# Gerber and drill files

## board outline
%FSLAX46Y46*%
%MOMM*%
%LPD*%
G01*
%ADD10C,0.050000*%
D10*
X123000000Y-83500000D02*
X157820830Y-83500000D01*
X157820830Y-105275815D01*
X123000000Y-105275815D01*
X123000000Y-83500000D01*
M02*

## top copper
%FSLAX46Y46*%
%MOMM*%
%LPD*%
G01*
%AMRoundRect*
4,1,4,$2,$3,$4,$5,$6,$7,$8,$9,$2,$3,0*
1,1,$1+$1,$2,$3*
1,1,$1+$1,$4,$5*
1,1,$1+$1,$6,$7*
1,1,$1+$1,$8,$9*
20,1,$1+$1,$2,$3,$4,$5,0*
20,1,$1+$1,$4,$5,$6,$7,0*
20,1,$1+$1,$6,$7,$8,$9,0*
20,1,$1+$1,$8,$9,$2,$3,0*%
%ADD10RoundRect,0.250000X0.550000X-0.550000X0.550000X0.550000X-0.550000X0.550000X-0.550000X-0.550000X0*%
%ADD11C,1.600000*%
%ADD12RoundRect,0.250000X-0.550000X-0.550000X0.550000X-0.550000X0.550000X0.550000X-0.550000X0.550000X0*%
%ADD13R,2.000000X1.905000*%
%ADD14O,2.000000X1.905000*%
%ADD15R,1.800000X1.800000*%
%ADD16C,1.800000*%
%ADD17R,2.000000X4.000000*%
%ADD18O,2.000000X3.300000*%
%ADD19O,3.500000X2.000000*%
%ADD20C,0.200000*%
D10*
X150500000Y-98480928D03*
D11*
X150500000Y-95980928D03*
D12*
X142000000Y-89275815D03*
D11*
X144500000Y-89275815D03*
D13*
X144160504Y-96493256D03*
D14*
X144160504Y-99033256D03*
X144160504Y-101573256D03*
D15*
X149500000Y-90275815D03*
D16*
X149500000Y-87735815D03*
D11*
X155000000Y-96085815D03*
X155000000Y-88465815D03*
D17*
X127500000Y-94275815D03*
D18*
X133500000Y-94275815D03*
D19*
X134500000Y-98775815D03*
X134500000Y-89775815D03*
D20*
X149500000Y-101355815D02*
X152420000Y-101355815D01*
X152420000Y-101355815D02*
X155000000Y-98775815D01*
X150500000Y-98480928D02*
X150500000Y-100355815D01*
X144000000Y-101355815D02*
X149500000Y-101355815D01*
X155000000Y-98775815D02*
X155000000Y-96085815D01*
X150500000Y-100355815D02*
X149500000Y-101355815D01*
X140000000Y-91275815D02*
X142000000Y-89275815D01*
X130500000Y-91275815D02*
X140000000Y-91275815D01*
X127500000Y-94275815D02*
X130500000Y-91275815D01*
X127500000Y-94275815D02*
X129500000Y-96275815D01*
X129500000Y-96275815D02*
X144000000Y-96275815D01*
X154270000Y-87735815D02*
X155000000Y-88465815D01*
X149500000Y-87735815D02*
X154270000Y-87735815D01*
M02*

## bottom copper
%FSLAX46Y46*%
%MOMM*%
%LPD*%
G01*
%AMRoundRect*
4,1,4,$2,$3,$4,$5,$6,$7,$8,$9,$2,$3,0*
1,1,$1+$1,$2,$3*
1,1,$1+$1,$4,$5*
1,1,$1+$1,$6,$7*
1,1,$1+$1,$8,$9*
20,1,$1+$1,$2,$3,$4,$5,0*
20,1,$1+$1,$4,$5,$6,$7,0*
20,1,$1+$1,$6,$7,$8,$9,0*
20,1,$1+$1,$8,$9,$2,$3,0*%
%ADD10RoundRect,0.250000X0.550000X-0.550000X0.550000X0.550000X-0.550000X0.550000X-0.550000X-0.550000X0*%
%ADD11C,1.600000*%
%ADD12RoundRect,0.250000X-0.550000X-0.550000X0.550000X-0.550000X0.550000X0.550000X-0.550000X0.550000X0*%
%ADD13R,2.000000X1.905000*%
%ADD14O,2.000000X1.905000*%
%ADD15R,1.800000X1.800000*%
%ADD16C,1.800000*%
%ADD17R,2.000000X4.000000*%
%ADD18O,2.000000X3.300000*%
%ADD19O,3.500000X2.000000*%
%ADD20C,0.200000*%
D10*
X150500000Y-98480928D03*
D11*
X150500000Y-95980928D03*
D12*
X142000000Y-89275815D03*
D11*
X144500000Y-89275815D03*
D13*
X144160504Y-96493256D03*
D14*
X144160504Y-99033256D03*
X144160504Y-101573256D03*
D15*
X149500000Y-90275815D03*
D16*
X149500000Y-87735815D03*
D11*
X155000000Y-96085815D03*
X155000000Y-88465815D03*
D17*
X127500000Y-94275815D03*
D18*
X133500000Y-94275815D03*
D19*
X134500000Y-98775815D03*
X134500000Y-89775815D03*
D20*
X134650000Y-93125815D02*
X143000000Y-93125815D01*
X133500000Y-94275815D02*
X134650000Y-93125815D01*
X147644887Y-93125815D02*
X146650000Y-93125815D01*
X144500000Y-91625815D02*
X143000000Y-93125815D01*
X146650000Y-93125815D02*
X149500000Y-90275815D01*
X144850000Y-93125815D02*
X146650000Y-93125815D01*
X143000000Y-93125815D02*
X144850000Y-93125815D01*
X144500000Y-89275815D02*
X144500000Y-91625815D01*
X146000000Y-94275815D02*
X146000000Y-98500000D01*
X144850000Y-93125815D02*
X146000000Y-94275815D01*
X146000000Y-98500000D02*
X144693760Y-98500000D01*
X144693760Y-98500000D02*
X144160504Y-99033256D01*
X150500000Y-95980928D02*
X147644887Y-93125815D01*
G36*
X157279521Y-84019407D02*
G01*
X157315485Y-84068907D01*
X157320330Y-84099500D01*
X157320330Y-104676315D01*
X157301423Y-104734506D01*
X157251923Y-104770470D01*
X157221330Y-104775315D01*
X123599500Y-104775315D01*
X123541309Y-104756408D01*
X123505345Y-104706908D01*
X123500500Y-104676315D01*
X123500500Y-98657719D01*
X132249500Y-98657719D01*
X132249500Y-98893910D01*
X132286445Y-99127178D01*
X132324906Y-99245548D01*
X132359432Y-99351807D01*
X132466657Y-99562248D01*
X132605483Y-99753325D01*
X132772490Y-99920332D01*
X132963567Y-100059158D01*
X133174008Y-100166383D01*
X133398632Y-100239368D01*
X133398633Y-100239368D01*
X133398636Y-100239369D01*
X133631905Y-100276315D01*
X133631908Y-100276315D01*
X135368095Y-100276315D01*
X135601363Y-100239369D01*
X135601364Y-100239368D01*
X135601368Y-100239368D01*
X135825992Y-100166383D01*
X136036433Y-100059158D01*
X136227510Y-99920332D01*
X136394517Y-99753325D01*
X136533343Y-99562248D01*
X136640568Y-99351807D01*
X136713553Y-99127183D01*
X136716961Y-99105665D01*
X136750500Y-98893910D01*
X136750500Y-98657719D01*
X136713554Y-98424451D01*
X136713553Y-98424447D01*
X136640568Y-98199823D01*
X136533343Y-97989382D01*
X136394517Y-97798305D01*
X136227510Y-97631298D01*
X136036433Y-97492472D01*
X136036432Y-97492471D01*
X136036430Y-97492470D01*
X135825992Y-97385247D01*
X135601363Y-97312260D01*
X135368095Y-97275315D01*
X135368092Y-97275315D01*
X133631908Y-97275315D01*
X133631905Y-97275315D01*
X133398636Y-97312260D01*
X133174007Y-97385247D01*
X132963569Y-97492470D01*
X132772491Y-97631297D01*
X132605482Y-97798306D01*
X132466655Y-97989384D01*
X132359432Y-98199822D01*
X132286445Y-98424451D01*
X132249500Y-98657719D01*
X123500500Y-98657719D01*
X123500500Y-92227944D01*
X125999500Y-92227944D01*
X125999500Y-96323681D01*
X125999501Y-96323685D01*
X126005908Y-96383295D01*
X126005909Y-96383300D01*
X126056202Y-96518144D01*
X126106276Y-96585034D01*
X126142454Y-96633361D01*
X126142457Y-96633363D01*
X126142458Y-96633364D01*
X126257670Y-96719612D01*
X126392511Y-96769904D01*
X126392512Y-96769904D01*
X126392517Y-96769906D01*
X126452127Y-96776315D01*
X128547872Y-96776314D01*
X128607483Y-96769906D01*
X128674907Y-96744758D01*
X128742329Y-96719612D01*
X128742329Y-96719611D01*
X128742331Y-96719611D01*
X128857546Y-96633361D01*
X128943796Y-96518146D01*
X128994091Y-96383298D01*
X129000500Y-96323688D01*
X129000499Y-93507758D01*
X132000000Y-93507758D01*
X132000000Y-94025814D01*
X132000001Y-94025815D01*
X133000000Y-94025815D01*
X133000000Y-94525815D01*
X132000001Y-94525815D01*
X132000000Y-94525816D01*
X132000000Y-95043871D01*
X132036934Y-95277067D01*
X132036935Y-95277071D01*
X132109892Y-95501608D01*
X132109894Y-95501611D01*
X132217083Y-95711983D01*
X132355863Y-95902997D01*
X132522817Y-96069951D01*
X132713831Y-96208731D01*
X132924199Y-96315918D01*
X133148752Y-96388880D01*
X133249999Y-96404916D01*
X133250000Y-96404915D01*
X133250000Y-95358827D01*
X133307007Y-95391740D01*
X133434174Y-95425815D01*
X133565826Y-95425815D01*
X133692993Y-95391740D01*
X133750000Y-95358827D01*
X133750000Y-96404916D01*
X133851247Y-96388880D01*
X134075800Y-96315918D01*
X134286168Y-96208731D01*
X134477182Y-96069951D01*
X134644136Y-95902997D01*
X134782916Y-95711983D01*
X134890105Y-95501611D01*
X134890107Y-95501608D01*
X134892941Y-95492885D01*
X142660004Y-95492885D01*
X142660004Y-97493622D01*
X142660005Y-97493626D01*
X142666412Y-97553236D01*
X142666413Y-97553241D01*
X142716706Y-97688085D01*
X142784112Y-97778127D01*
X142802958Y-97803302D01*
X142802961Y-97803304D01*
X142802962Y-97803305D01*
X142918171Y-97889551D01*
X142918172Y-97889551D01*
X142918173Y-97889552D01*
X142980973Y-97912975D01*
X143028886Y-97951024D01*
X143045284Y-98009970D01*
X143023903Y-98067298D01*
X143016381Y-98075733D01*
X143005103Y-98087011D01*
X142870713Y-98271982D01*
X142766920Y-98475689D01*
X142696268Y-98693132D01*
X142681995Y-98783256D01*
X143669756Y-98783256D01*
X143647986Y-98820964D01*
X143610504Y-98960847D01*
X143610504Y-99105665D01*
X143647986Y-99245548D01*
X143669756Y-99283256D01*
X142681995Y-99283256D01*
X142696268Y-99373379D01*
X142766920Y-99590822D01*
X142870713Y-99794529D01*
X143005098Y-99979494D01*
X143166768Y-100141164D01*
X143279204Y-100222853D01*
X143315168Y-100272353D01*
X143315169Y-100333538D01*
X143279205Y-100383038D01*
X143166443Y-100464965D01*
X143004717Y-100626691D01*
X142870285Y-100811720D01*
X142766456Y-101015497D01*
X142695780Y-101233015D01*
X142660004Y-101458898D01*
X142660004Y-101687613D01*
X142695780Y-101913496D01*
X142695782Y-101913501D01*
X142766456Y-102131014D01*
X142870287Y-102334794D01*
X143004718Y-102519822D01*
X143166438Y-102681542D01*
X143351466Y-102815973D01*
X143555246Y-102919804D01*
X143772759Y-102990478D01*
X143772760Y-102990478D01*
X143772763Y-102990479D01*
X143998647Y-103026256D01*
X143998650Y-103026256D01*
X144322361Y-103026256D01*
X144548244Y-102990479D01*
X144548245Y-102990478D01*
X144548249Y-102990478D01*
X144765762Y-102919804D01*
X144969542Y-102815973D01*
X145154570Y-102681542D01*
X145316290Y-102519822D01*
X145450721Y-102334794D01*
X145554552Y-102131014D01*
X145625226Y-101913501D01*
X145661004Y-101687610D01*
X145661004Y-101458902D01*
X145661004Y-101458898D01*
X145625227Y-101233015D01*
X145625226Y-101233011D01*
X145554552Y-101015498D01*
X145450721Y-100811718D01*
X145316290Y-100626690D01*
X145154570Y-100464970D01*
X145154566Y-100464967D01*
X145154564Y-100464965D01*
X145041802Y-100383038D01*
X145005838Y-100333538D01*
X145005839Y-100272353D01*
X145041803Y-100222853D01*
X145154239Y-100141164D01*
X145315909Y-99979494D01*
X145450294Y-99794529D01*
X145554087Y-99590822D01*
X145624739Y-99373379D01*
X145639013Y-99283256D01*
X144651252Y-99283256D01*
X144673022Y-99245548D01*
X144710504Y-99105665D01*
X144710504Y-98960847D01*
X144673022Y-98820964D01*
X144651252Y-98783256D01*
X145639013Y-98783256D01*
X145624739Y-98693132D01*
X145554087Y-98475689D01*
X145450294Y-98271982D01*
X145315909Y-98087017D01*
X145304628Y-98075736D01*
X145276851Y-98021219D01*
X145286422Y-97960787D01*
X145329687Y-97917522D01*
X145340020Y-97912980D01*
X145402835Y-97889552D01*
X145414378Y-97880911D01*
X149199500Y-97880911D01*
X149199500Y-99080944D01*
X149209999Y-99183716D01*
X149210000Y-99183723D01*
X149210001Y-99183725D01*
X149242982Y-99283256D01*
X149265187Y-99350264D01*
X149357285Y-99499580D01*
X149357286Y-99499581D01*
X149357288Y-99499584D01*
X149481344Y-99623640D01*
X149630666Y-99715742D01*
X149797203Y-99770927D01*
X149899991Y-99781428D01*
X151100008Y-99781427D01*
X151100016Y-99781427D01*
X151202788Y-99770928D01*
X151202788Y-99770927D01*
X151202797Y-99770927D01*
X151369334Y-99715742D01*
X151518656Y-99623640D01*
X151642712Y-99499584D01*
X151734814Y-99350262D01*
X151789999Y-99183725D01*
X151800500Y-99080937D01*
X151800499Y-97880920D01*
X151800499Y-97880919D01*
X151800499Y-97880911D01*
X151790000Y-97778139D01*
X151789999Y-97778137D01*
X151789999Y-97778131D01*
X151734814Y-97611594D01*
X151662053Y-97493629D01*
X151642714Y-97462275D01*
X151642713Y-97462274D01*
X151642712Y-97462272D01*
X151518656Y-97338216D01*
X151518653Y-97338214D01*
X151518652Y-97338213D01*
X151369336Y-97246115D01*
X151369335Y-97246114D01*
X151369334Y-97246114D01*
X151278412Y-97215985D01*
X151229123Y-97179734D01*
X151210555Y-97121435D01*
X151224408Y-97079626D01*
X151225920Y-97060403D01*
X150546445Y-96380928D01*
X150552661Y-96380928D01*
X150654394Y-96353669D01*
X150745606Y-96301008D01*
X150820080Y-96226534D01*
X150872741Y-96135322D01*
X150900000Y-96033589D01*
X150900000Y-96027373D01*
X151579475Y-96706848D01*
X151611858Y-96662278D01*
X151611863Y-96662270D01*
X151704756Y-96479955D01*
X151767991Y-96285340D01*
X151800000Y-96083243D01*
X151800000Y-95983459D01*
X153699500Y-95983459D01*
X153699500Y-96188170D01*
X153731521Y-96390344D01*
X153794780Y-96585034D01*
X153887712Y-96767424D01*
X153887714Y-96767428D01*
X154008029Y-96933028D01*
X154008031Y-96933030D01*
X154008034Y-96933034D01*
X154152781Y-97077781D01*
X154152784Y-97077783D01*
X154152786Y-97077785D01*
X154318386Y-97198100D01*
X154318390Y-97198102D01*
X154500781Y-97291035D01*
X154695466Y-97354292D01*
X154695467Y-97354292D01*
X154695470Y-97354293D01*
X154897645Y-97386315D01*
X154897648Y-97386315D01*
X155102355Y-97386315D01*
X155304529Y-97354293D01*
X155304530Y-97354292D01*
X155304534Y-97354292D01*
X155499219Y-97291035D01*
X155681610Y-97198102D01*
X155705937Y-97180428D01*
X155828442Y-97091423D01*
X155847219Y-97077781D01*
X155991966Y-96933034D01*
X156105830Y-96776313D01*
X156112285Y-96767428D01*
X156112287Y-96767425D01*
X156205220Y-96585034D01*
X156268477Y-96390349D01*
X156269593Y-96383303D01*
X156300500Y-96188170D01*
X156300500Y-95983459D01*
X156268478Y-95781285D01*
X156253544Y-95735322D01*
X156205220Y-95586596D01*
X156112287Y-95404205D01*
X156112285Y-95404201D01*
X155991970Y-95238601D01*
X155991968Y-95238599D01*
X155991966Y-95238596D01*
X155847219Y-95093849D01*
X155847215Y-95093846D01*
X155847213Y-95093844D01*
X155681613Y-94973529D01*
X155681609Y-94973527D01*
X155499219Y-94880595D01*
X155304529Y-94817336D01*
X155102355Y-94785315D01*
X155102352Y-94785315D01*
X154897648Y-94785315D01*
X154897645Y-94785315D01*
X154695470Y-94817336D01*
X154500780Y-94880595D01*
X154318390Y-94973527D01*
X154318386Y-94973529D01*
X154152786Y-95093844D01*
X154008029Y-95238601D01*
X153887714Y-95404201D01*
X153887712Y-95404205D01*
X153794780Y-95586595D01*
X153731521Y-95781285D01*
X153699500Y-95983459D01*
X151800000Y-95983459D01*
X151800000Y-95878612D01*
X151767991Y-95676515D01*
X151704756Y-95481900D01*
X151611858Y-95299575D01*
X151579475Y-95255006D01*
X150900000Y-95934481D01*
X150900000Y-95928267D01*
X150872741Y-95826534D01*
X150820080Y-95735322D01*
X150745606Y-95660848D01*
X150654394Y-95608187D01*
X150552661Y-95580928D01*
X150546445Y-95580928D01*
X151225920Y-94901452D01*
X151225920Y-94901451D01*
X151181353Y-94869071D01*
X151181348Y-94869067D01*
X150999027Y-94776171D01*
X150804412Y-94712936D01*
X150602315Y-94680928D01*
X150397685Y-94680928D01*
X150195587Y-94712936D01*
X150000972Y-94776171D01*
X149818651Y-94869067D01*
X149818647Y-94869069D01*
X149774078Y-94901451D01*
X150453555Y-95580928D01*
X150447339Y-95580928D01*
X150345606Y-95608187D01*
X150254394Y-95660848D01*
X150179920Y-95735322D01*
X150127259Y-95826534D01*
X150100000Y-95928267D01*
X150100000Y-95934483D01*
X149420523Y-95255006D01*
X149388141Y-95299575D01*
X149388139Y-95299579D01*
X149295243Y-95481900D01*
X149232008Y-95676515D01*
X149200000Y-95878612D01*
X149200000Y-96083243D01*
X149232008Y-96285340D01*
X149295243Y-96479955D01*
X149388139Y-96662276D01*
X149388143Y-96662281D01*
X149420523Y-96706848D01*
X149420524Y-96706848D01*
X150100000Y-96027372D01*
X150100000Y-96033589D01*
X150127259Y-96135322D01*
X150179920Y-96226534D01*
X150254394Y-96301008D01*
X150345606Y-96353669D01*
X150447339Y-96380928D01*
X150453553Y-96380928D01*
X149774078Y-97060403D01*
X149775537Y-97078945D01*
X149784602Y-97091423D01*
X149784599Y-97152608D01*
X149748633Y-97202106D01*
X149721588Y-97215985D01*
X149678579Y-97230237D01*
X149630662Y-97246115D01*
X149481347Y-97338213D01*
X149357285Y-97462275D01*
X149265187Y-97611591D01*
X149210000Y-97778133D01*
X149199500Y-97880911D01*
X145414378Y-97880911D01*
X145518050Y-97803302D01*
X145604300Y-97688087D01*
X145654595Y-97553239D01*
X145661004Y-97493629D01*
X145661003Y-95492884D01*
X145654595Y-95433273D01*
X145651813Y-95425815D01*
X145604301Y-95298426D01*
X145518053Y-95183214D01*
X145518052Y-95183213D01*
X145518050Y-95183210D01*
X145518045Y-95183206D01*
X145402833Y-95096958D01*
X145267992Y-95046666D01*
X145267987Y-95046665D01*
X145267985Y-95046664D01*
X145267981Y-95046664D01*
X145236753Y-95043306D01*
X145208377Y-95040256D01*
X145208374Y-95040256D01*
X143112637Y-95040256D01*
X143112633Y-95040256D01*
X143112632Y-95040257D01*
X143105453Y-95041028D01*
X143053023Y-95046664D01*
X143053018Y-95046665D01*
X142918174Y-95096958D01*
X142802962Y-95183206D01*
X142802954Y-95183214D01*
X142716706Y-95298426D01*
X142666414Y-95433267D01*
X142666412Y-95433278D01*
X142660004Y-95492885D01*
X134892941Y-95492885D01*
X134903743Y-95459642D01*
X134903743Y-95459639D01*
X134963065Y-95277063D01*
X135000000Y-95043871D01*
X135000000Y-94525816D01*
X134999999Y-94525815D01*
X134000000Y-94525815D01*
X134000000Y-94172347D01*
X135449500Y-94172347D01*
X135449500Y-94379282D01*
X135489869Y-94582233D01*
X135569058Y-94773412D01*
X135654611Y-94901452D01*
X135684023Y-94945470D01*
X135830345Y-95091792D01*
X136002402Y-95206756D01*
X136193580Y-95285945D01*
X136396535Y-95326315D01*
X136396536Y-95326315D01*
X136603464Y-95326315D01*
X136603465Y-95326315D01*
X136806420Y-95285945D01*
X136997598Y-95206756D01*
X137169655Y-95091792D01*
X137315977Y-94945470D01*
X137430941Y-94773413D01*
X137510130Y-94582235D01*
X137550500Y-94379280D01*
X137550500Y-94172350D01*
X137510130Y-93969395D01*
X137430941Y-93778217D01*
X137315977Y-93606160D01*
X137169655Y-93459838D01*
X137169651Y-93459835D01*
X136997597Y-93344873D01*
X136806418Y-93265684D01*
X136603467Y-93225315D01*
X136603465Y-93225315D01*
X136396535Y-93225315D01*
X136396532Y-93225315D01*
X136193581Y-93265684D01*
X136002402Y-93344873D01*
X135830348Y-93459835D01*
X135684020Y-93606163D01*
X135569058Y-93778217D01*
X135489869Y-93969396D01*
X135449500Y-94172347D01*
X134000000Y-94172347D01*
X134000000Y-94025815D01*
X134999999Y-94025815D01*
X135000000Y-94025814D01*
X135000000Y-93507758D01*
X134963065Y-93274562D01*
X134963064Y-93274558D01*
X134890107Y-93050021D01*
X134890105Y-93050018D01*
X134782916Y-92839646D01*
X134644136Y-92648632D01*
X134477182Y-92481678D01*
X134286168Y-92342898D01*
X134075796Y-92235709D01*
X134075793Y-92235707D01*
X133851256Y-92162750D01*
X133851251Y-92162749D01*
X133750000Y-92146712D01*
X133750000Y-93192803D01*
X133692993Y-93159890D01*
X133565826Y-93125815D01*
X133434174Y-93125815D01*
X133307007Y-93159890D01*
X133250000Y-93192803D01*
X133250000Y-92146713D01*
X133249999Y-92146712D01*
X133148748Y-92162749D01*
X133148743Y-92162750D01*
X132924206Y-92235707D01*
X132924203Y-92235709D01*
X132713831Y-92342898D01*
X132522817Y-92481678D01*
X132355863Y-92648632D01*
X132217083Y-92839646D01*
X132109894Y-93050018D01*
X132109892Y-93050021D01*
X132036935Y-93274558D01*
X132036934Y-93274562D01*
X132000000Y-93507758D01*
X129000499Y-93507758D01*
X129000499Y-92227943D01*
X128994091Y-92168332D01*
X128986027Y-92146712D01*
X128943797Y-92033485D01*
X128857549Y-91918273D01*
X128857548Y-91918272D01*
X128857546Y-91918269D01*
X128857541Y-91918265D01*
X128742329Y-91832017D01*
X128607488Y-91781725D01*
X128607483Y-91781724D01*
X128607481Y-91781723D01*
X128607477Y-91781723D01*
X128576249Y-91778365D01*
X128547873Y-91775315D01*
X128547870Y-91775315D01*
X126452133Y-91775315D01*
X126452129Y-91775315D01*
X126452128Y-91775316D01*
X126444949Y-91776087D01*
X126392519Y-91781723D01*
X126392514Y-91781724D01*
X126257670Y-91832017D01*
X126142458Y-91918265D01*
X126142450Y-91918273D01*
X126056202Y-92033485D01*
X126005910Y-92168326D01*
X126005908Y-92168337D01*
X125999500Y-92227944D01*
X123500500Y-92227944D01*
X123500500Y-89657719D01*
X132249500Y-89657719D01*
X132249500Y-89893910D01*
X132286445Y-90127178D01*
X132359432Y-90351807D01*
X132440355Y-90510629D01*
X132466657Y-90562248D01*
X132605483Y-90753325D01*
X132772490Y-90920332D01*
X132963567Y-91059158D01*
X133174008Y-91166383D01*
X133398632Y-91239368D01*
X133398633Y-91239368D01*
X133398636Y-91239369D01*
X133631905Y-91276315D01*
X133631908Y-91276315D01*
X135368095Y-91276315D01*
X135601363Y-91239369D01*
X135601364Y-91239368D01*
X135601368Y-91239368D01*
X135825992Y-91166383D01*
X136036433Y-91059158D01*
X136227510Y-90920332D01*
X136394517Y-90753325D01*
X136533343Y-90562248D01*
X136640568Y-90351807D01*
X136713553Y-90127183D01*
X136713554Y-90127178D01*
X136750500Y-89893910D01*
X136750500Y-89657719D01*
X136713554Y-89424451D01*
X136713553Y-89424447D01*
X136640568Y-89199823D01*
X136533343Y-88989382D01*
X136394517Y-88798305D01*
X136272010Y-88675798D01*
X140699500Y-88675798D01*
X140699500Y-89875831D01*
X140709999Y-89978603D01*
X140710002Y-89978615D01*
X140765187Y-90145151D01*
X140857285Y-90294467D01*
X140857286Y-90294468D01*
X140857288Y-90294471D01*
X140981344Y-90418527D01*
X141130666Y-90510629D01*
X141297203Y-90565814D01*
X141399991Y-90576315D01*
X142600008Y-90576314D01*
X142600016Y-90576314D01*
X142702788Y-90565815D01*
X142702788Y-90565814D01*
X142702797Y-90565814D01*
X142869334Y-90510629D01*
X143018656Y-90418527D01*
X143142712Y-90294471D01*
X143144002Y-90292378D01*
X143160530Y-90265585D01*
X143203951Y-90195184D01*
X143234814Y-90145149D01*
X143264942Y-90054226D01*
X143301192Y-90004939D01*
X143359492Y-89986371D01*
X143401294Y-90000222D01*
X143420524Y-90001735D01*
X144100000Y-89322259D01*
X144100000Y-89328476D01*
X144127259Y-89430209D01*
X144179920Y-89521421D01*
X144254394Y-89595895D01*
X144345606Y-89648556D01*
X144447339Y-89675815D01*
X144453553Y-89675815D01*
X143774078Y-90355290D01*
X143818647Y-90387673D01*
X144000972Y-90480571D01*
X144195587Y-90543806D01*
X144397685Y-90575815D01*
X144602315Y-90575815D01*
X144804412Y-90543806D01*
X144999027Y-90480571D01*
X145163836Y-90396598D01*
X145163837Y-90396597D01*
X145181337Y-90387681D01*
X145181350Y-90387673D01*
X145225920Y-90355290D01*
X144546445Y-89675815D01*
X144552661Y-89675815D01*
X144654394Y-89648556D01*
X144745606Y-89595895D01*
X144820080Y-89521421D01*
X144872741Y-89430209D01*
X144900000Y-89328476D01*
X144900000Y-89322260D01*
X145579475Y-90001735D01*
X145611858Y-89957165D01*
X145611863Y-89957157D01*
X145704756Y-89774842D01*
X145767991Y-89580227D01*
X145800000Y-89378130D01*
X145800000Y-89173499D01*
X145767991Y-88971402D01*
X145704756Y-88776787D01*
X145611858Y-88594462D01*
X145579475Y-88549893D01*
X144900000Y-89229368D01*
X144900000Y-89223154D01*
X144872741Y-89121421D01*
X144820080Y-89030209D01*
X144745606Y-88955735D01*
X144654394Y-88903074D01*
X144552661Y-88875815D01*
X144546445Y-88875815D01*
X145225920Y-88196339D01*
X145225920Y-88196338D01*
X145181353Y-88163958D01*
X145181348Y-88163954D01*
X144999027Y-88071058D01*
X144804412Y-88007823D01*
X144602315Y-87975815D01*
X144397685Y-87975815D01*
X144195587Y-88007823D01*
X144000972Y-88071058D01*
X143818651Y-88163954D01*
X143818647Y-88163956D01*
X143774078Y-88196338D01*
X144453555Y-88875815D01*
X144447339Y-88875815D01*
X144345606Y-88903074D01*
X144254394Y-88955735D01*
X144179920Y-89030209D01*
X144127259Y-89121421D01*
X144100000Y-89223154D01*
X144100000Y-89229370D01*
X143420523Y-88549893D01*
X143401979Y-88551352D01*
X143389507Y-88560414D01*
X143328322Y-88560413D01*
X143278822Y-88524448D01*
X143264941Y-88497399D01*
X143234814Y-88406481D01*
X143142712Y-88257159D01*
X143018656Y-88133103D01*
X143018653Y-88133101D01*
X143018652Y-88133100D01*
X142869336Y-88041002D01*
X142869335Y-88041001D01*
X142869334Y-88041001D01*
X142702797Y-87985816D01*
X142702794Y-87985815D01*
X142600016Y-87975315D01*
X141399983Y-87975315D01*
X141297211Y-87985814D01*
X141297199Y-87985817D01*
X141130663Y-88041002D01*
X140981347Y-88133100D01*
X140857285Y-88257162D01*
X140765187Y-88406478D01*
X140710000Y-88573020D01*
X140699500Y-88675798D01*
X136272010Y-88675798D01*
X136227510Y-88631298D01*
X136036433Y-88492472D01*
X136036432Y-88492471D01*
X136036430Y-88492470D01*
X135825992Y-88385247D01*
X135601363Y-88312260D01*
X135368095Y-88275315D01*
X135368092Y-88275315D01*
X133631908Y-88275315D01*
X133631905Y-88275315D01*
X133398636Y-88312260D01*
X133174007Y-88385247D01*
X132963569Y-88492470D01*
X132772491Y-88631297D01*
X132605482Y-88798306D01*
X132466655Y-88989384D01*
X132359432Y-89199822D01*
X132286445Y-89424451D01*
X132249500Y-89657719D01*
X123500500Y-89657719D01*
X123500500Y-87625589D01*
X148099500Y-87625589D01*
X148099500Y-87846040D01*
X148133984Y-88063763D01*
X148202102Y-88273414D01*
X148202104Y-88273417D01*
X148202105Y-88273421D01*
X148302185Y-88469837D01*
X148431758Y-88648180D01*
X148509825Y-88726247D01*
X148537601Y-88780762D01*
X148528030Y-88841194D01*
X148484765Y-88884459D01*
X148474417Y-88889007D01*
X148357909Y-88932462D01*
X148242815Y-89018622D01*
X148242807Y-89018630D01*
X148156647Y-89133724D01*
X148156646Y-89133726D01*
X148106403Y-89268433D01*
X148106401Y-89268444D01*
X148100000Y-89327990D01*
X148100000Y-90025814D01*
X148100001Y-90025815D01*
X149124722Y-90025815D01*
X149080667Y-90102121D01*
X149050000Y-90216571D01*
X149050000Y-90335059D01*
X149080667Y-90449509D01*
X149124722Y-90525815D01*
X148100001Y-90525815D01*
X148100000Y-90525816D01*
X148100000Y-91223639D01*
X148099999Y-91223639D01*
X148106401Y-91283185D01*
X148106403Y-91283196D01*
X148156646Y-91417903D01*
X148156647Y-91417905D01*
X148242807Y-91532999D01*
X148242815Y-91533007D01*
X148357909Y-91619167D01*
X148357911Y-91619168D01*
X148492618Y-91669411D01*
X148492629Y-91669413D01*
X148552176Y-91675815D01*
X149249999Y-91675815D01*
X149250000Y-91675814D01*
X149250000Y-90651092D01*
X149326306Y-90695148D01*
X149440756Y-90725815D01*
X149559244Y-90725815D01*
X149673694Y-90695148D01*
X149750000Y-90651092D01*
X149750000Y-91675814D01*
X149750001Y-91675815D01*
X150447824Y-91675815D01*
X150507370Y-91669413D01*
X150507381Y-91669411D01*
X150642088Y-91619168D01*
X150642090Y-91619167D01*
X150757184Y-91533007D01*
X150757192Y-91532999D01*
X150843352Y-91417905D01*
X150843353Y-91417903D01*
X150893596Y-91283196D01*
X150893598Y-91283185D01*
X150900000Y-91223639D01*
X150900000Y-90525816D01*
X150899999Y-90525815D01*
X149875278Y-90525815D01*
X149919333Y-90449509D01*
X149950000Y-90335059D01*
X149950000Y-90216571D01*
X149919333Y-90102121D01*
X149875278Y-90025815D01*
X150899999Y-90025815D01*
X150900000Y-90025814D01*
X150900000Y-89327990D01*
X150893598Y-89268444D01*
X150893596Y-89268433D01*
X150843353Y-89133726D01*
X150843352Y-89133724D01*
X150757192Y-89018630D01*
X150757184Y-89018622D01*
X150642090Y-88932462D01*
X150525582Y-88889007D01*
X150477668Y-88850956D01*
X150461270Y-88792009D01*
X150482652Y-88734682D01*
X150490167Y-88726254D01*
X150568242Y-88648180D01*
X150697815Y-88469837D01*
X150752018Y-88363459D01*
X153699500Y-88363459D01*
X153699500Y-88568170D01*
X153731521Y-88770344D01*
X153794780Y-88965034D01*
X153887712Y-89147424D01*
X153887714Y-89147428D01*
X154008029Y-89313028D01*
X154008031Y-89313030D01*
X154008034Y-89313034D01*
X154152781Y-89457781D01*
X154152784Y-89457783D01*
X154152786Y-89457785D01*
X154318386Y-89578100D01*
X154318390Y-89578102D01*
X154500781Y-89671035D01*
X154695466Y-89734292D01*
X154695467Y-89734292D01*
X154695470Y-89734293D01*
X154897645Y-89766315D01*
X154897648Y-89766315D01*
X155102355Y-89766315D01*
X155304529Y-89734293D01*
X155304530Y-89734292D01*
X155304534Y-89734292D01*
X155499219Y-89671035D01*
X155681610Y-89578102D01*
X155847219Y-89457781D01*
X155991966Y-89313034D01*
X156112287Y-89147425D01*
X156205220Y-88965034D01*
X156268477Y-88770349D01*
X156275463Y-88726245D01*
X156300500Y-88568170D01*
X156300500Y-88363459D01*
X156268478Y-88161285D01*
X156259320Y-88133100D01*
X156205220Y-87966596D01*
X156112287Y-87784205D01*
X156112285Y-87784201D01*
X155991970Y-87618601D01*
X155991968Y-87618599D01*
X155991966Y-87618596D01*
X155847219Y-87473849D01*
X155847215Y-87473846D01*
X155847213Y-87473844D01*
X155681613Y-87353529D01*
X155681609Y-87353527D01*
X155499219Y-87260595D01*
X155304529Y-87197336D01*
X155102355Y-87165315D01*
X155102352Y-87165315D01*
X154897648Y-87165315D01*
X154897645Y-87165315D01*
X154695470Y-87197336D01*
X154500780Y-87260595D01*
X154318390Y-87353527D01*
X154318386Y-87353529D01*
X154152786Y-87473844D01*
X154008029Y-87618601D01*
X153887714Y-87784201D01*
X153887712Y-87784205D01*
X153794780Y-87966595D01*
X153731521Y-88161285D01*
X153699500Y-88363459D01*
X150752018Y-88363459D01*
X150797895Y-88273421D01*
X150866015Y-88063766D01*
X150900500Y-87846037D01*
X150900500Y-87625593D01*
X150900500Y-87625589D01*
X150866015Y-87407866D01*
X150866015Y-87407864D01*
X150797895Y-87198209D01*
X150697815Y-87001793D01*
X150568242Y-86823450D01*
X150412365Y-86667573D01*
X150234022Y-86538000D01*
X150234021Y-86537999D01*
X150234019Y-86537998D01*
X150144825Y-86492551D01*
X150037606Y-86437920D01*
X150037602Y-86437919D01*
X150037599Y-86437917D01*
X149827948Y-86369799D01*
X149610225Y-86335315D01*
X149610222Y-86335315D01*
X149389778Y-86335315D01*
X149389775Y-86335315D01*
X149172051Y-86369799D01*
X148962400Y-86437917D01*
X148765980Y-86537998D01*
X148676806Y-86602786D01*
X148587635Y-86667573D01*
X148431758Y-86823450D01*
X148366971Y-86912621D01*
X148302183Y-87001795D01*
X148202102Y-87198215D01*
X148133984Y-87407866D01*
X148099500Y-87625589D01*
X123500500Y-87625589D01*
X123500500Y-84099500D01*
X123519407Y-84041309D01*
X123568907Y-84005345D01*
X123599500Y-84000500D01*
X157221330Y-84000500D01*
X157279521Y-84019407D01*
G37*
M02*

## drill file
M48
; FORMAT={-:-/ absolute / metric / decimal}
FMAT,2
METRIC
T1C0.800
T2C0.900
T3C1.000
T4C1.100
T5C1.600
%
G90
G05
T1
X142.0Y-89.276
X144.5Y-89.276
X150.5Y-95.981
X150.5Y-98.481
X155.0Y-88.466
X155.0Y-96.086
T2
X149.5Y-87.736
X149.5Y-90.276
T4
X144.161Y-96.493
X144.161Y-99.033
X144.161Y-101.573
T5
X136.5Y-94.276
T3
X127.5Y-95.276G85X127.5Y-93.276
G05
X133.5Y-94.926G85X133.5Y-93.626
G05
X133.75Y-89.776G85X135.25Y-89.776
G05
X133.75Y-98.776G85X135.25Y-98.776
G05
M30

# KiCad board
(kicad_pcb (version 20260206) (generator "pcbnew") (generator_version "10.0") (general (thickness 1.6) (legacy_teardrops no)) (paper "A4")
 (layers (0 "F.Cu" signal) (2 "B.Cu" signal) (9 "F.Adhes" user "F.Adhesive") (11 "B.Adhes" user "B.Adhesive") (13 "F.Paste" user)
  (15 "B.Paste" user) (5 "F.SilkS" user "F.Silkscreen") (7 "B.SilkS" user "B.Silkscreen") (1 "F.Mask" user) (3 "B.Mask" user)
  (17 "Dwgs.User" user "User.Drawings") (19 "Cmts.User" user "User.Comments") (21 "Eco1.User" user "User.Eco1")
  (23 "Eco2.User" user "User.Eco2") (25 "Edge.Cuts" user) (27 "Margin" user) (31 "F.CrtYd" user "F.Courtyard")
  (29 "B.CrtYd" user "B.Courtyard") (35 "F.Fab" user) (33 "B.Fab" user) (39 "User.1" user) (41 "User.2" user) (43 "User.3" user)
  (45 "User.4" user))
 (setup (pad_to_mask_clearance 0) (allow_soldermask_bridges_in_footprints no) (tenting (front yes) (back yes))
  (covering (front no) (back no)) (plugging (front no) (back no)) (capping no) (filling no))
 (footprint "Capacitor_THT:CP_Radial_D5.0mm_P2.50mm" (layer "F.Cu") (at 150.5 98.480928 90)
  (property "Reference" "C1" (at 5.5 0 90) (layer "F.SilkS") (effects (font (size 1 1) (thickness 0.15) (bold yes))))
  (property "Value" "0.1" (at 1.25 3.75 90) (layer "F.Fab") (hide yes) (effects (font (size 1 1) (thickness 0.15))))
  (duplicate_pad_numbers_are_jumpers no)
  (pad "1" thru_hole roundrect (at 0 0 90) (size 1.6 1.6) (drill 0.8) (layers "*.Cu" "*.Mask") (remove_unused_layers no)
   (roundrect_rratio 0.15625) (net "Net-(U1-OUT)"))
  (pad "2" thru_hole circle (at 2.5 0 90) (size 1.6 1.6) (drill 0.8) (layers "*.Cu" "*.Mask") (remove_unused_layers no) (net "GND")))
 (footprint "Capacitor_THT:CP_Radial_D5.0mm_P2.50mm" (layer "F.Cu") (at 142 89.275815)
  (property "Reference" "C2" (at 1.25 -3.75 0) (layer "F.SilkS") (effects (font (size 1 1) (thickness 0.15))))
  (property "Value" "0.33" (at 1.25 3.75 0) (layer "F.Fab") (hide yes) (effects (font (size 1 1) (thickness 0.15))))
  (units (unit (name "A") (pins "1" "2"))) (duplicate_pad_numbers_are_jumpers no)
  (pad "1" thru_hole roundrect (at 0 0) (size 1.6 1.6) (drill 0.8) (layers "*.Cu" "*.Mask") (remove_unused_layers no)
   (roundrect_rratio 0.15625) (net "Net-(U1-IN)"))
  (pad "2" thru_hole circle (at 2.5 0) (size 1.6 1.6) (drill 0.8) (layers "*.Cu" "*.Mask") (remove_unused_layers no) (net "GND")))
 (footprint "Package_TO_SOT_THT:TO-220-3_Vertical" (layer "F.Cu") (at 144.160504 96.493256 -90)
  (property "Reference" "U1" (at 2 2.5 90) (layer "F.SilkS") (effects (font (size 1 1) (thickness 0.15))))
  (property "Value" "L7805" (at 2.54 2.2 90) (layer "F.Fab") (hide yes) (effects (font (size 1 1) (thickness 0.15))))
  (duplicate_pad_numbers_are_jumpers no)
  (pad "1" thru_hole rect (at 0 0 270) (size 1.905 2) (drill 1.1) (layers "*.Cu" "*.Mask") (remove_unused_layers no) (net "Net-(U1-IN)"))
  (pad "2" thru_hole oval (at 2.54 0 270) (size 1.905 2) (drill 1.1) (layers "*.Cu" "*.Mask") (remove_unused_layers no) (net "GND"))
  (pad "3" thru_hole oval (at 5.08 0 270) (size 1.905 2) (drill 1.1) (layers "*.Cu" "*.Mask") (remove_unused_layers no) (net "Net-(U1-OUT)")))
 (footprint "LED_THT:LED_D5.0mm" (layer "F.Cu") (at 149.5 90.275815 90)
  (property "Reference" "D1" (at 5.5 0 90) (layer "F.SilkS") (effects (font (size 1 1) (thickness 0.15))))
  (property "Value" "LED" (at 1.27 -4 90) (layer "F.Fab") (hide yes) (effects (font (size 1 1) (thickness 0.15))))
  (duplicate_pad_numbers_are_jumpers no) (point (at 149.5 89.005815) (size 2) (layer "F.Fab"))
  (pad "1" thru_hole rect (at 0 0 90) (size 1.8 1.8) (drill 0.9) (layers "*.Cu" "*.Mask") (remove_unused_layers no) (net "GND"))
  (pad "2" thru_hole circle (at 2.54 0 90) (size 1.8 1.8) (drill 0.9) (layers "*.Cu" "*.Mask") (remove_unused_layers no) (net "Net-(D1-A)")))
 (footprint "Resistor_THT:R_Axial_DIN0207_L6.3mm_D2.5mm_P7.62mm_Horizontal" (layer "F.Cu") (at 155 96.085815 90)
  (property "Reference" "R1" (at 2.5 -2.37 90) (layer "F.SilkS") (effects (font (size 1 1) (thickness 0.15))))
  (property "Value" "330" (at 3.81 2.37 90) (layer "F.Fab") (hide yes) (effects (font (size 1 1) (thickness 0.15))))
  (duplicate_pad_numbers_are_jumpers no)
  (pad "1" thru_hole circle (at 0 0 90) (size 1.6 1.6) (drill 0.8) (layers "*.Cu" "*.Mask") (remove_unused_layers no) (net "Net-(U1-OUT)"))
  (pad "2" thru_hole circle (at 7.62 0 90) (size 1.6 1.6) (drill 0.8) (layers "*.Cu" "*.Mask") (remove_unused_layers no) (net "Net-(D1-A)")))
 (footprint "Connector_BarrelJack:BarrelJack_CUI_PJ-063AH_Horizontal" (layer "F.Cu") (at 127.5 94.275815 90)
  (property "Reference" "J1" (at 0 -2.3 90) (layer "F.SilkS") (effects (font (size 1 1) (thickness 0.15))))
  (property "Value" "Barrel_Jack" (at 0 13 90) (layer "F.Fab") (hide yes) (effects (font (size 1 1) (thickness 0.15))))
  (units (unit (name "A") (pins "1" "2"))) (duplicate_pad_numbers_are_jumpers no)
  (pad "" np_thru_hole circle (at 0 9 90) (size 1.6 1.6) (drill 1.6) (layers "*.Cu" "*.Mask"))
  (pad "1" thru_hole rect (at 0 0 90) (size 4 2) (drill oval 3 1) (layers "*.Cu" "*.Mask") (remove_unused_layers no) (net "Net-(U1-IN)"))
  (pad "2" thru_hole oval (at 0 6 90) (size 3.3 2) (drill oval 2.3 1) (layers "*.Cu" "*.Mask") (remove_unused_layers no) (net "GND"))
  (pad "MP" thru_hole oval (at -4.5 7 90) (size 2 3.5) (drill oval 1 2.5) (layers "*.Cu" "*.Mask") (remove_unused_layers no))
  (pad "MP" thru_hole oval (at 4.5 7 90) (size 2 3.5) (drill oval 1 2.5) (layers "*.Cu" "*.Mask") (remove_unused_layers no)))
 (gr_rect (start 123 83.5) (end 157.82083 105.275815) (stroke (width 0.05) (type default)) (fill no) (layer "Edge.Cuts"))
 (segment (start 149.5 101.355815) (end 152.42 101.355815) (width 0.2) (layer "F.Cu") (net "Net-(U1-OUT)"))
 (segment (start 152.42 101.355815) (end 155 98.775815) (width 0.2) (layer "F.Cu") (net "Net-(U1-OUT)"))
 (segment (start 150.5 98.480928) (end 150.5 100.355815) (width 0.2) (layer "F.Cu") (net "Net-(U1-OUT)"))
 (segment (start 144 101.355815) (end 149.5 101.355815) (width 0.2) (layer "F.Cu") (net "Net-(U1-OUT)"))
 (segment (start 155 98.775815) (end 155 96.085815) (width 0.2) (layer "F.Cu") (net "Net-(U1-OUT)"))
 (segment (start 150.5 100.355815) (end 149.5 101.355815) (width 0.2) (layer "F.Cu") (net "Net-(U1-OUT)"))
 (segment (start 134.65 93.125815) (end 143 93.125815) (width 0.2) (layer "B.Cu") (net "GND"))
 (segment (start 133.5 94.275815) (end 134.65 93.125815) (width 0.2) (layer "B.Cu") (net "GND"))
 (segment (start 147.644887 93.125815) (end 146.65 93.125815) (width 0.2) (layer "B.Cu") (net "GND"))
 (segment (start 144.5 91.625815) (end 143 93.125815) (width 0.2) (layer "B.Cu") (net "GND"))
 (segment (start 146.65 93.125815) (end 149.5 90.275815) (width 0.2) (layer "B.Cu") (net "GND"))
 (segment (start 144.85 93.125815) (end 146.65 93.125815) (width 0.2) (layer "B.Cu") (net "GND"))
 (segment (start 143 93.125815) (end 144.85 93.125815) (width 0.2) (layer "B.Cu") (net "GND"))
 (segment (start 144.5 89.275815) (end 144.5 91.625815) (width 0.2) (layer "B.Cu") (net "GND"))
 (segment (start 146 94.275815) (end 146 98.5) (width 0.2) (layer "B.Cu") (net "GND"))
 (segment (start 144.85 93.125815) (end 146 94.275815) (width 0.2) (layer "B.Cu") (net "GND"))
 (segment (start 146 98.5) (end 144.69376 98.5) (width 0.2) (layer "B.Cu") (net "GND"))
 (segment (start 144.69376 98.5) (end 144.160504 99.033256) (width 0.2) (layer "B.Cu") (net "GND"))
 (segment (start 150.5 95.980928) (end 147.644887 93.125815) (width 0.2) (layer "B.Cu") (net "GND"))
 (segment (start 140 91.275815) (end 142 89.275815) (width 0.2) (layer "F.Cu") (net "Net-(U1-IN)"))
 (segment (start 130.5 91.275815) (end 140 91.275815) (width 0.2) (layer "F.Cu") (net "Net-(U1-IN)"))
 (segment (start 127.5 94.275815) (end 130.5 91.275815) (width 0.2) (layer "F.Cu") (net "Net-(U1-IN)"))
 (segment (start 127.5 94.275815) (end 129.5 96.275815) (width 0.2) (layer "F.Cu") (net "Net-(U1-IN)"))
 (segment (start 129.5 96.275815) (end 144 96.275815) (width 0.2) (layer "F.Cu") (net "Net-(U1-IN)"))
 (segment (start 154.27 87.735815) (end 155 88.465815) (width 0.2) (layer "F.Cu") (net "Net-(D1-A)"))
 (segment (start 149.5 87.735815) (end 154.27 87.735815) (width 0.2) (layer "F.Cu") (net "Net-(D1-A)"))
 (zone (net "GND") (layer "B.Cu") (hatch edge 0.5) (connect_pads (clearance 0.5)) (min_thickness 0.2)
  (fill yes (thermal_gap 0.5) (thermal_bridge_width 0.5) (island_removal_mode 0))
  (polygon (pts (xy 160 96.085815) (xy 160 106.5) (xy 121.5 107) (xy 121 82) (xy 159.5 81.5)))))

